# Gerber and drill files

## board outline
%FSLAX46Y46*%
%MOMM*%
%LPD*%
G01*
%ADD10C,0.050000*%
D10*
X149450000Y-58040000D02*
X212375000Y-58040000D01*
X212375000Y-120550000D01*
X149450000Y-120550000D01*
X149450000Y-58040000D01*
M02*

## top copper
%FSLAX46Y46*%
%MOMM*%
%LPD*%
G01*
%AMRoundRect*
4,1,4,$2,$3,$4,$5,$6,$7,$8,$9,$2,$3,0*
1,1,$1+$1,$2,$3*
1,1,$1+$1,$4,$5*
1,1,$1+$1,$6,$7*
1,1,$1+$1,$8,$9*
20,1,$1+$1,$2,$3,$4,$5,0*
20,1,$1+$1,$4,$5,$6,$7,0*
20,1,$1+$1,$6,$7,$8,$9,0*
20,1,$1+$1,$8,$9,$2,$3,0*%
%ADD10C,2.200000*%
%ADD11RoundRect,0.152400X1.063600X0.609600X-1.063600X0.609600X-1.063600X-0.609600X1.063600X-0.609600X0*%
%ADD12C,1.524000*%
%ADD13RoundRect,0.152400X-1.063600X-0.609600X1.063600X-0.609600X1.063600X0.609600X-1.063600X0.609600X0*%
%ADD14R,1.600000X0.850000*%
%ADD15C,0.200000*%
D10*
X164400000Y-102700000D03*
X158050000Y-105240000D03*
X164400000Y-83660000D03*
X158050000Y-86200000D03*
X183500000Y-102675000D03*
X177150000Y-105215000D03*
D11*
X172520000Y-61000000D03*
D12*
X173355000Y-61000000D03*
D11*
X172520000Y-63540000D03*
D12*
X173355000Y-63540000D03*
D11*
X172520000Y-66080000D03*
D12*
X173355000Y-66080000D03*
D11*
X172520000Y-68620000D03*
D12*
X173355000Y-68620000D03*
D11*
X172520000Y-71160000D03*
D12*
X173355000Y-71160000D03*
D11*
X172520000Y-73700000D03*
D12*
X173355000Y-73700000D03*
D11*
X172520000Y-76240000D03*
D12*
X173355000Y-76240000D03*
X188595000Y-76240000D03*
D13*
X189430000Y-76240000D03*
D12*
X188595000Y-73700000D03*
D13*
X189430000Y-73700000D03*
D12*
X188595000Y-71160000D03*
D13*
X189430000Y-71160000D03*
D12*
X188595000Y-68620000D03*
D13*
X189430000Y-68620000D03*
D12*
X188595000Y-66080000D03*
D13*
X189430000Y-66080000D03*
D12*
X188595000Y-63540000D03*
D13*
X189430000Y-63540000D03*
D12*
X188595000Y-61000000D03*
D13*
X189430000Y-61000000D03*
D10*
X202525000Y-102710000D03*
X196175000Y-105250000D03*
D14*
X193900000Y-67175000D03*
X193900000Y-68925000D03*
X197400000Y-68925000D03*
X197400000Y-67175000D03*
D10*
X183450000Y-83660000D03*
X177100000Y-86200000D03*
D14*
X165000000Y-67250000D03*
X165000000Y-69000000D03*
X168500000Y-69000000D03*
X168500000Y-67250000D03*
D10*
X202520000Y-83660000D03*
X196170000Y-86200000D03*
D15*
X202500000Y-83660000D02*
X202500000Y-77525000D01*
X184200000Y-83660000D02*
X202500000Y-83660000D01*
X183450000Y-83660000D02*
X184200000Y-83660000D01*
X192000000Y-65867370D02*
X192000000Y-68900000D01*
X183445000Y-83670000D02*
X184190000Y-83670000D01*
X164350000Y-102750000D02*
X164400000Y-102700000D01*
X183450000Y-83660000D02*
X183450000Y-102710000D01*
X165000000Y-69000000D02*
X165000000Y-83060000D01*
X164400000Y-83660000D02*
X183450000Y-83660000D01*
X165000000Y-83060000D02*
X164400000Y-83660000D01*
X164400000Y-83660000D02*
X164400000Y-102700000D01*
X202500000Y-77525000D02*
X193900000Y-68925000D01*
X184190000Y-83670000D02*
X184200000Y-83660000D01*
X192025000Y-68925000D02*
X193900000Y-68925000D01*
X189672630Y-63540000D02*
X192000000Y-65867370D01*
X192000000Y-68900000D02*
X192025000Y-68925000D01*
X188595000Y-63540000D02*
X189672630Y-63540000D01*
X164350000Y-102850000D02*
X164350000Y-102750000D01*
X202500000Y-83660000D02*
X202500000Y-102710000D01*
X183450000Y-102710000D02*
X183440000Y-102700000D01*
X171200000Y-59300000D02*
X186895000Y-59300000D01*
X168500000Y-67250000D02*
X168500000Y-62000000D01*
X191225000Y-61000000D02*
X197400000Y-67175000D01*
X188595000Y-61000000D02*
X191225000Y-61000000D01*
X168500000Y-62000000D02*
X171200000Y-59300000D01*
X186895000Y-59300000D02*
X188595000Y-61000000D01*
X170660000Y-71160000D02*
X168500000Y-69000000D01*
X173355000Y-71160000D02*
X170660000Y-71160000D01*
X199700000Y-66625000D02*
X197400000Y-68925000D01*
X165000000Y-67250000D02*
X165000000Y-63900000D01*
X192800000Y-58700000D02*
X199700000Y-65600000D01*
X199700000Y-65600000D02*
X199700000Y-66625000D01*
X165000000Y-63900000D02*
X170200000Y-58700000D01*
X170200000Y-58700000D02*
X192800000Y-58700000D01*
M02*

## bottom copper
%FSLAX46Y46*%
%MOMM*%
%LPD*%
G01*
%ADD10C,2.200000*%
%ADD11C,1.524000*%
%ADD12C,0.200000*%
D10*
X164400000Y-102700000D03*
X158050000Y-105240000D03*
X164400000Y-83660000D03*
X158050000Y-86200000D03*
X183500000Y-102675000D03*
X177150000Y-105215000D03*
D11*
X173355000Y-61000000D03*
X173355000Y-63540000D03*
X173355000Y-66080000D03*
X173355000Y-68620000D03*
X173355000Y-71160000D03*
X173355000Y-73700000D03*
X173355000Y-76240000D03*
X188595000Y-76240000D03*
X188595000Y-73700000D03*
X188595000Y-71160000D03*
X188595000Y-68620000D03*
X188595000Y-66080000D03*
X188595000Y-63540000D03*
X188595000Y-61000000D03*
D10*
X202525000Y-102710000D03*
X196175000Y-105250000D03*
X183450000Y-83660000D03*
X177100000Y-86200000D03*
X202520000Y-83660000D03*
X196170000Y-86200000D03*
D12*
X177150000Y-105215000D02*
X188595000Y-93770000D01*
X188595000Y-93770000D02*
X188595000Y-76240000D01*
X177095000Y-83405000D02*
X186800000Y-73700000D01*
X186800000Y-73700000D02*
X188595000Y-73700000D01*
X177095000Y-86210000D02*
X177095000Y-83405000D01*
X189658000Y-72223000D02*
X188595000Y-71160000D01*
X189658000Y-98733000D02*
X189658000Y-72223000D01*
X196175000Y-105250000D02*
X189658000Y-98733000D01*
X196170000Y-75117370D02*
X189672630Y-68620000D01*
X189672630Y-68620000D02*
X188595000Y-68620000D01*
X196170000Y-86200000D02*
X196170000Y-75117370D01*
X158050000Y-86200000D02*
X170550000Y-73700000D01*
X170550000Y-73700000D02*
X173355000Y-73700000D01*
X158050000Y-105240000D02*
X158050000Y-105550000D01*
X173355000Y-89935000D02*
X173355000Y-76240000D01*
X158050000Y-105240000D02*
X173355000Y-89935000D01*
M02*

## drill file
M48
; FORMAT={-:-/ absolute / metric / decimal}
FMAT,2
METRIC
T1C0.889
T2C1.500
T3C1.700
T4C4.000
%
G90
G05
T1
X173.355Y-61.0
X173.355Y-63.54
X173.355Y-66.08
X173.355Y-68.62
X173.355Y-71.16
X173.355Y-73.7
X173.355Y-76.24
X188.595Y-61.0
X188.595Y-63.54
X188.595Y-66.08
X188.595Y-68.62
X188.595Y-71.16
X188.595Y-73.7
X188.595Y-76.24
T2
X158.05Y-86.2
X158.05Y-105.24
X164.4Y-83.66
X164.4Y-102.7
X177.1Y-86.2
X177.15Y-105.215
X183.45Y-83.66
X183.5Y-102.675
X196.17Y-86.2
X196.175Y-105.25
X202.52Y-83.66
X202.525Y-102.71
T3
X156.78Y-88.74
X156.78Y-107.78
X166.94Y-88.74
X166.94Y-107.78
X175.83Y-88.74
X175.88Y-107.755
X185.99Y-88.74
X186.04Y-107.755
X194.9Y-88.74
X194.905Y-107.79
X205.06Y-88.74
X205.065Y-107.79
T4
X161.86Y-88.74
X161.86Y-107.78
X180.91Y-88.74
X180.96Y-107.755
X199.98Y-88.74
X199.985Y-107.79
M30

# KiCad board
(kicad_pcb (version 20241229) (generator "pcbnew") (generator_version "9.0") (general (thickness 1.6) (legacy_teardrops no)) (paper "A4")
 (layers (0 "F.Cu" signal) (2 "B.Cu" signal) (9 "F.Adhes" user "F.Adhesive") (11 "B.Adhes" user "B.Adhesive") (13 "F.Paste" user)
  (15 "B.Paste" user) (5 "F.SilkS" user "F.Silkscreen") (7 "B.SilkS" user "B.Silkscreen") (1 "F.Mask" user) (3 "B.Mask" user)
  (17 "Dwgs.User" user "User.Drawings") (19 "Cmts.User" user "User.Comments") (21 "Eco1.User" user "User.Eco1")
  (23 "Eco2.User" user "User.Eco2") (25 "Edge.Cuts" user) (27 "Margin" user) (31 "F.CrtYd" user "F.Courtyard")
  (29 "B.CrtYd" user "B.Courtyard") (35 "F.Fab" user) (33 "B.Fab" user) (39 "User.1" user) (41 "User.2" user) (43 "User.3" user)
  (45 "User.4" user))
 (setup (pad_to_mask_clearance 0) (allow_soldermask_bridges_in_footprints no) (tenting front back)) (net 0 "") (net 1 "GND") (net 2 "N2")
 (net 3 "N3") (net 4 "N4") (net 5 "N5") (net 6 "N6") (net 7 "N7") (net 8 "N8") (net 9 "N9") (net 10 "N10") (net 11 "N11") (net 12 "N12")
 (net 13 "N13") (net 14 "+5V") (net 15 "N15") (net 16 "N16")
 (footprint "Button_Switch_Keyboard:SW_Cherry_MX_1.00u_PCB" (layer "F.Cu") (at 164.4 102.7)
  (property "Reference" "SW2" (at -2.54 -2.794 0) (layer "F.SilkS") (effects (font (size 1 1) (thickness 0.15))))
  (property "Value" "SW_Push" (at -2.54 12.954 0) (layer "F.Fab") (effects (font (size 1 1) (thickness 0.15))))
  (pad "" np_thru_hole circle (at -7.62 5.08) (size 1.7 1.7) (drill 1.7) (layers "*.Cu" "*.Mask"))
  (pad "" np_thru_hole circle (at -2.54 5.08) (size 4 4) (drill 4) (layers "*.Cu" "*.Mask"))
  (pad "" np_thru_hole circle (at 2.54 5.08) (size 1.7 1.7) (drill 1.7) (layers "*.Cu" "*.Mask"))
  (pad "1" thru_hole circle (at 0 0) (size 2.2 2.2) (drill 1.5) (layers "*.Cu" "*.Mask") (remove_unused_layers no) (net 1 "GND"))
  (pad "2" thru_hole circle (at -6.35 2.54) (size 2.2 2.2) (drill 1.5) (layers "*.Cu" "*.Mask") (remove_unused_layers no) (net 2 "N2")))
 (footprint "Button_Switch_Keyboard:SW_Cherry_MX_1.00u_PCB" (layer "F.Cu") (at 164.4 83.66)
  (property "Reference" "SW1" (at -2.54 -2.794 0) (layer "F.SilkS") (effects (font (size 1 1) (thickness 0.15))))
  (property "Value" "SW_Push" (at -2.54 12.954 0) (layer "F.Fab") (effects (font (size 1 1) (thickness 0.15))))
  (pad "" np_thru_hole circle (at -7.62 5.08) (size 1.7 1.7) (drill 1.7) (layers "*.Cu" "*.Mask"))
  (pad "" np_thru_hole circle (at -2.54 5.08) (size 4 4) (drill 4) (layers "*.Cu" "*.Mask"))
  (pad "" np_thru_hole circle (at 2.54 5.08) (size 1.7 1.7) (drill 1.7) (layers "*.Cu" "*.Mask"))
  (pad "1" thru_hole circle (at 0 0) (size 2.2 2.2) (drill 1.5) (layers "*.Cu" "*.Mask") (remove_unused_layers no) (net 1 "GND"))
  (pad "2" thru_hole circle (at -6.35 2.54) (size 2.2 2.2) (drill 1.5) (layers "*.Cu" "*.Mask") (remove_unused_layers no) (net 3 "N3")))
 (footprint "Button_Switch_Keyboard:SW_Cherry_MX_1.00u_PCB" (layer "F.Cu") (at 183.5 102.675)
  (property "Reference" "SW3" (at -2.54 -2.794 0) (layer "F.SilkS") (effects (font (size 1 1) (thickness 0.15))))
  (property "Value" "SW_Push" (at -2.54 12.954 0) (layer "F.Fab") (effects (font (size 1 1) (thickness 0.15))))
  (pad "" np_thru_hole circle (at -7.62 5.08) (size 1.7 1.7) (drill 1.7) (layers "*.Cu" "*.Mask"))
  (pad "" np_thru_hole circle (at -2.54 5.08) (size 4 4) (drill 4) (layers "*.Cu" "*.Mask"))
  (pad "" np_thru_hole circle (at 2.54 5.08) (size 1.7 1.7) (drill 1.7) (layers "*.Cu" "*.Mask"))
  (pad "1" thru_hole circle (at 0 0) (size 2.2 2.2) (drill 1.5) (layers "*.Cu" "*.Mask") (remove_unused_layers no) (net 1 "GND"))
  (pad "2" thru_hole circle (at -6.35 2.54) (size 2.2 2.2) (drill 1.5) (layers "*.Cu" "*.Mask") (remove_unused_layers no) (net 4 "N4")))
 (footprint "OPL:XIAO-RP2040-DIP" (layer "F.Cu") (at 180.975 68.62)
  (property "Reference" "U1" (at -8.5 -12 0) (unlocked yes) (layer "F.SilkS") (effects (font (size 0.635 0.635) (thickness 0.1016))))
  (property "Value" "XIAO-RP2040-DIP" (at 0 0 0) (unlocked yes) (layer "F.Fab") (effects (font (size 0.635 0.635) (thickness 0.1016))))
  (pad "1" smd roundrect (at -8.455 -7.62 180) (size 2.432 1.524) (layers "F.Cu" "F.Mask") (roundrect_rratio 0.1) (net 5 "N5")
   (thermal_bridge_angle 45))
  (pad "1" thru_hole circle (at -7.62 -7.62 180) (size 1.524 1.524) (drill 0.889) (layers "*.Cu" "*.Mask") (remove_unused_layers no)
   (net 5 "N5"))
  (pad "2" smd roundrect (at -8.455 -5.08 180) (size 2.432 1.524) (layers "F.Cu" "F.Mask") (roundrect_rratio 0.1) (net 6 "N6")
   (thermal_bridge_angle 45))
  (pad "2" thru_hole circle (at -7.62 -5.08 180) (size 1.524 1.524) (drill 0.889) (layers "*.Cu" "*.Mask") (remove_unused_layers no)
   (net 6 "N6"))
  (pad "3" smd roundrect (at -8.455 -2.54 180) (size 2.432 1.524) (layers "F.Cu" "F.Mask") (roundrect_rratio 0.1) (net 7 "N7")
   (thermal_bridge_angle 45))
  (pad "3" thru_hole circle (at -7.62 -2.54 180) (size 1.524 1.524) (drill 0.889) (layers "*.Cu" "*.Mask") (remove_unused_layers no)
   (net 7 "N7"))
  (pad "4" smd roundrect (at -8.455 0 180) (size 2.432 1.524) (layers "F.Cu" "F.Mask") (roundrect_rratio 0.1) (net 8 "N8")
   (thermal_bridge_angle 45))
  (pad "4" thru_hole circle (at -7.62 0 180) (size 1.524 1.524) (drill 0.889) (layers "*.Cu" "*.Mask") (remove_unused_layers no)
   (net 8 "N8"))
  (pad "5" smd roundrect (at -8.455 2.54 180) (size 2.432 1.524) (layers "F.Cu" "F.Mask") (roundrect_rratio 0.1) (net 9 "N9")
   (thermal_bridge_angle 45))
  (pad "5" thru_hole circle (at -7.62 2.54 180) (size 1.524 1.524) (drill 0.889) (layers "*.Cu" "*.Mask") (remove_unused_layers no)
   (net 9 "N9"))
  (pad "6" smd roundrect (at -8.455 5.08 180) (size 2.432 1.524) (layers "F.Cu" "F.Mask") (roundrect_rratio 0.1) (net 3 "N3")
   (thermal_bridge_angle 45))
  (pad "6" thru_hole circle (at -7.62 5.08 180) (size 1.524 1.524) (drill 0.889) (layers "*.Cu" "*.Mask") (remove_unused_layers no)
   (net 3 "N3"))
  (pad "7" smd roundrect (at -8.455 7.62 180) (size 2.432 1.524) (layers "F.Cu" "F.Mask") (roundrect_rratio 0.1) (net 2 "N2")
   (thermal_bridge_angle 45))
  (pad "7" thru_hole circle (at -7.62 7.62 180) (size 1.524 1.524) (drill 0.889) (layers "*.Cu" "*.Mask") (remove_unused_layers no)
   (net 2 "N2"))
  (pad "8" thru_hole circle (at 7.62 7.62) (size 1.524 1.524) (drill 0.889) (layers "*.Cu" "*.Mask") (remove_unused_layers no) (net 4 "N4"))
  (pad "8" smd roundrect (at 8.455 7.62) (size 2.432 1.524) (layers "F.Cu" "F.Mask") (roundrect_rratio 0.1) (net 4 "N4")
   (thermal_bridge_angle 45))
  (pad "9" thru_hole circle (at 7.62 5.08) (size 1.524 1.524) (drill 0.889) (layers "*.Cu" "*.Mask") (remove_unused_layers no)
   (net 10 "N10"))
  (pad "9" smd roundrect (at 8.455 5.08) (size 2.432 1.524) (layers "F.Cu" "F.Mask") (roundrect_rratio 0.1) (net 10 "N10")
   (thermal_bridge_angle 45))
  (pad "10" thru_hole circle (at 7.62 2.54) (size 1.524 1.524) (drill 0.889) (layers "*.Cu" "*.Mask") (remove_unused_layers no)
   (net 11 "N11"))
  (pad "10" smd roundrect (at 8.455 2.54) (size 2.432 1.524) (layers "F.Cu" "F.Mask") (roundrect_rratio 0.1) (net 11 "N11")
   (thermal_bridge_angle 45))
  (pad "11" thru_hole circle (at 7.62 0) (size 1.524 1.524) (drill 0.889) (layers "*.Cu" "*.Mask") (remove_unused_layers no) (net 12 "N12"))
  (pad "11" smd roundrect (at 8.455 0) (size 2.432 1.524) (layers "F.Cu" "F.Mask") (roundrect_rratio 0.1) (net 12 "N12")
   (thermal_bridge_angle 45))
  (pad "12" thru_hole circle (at 7.62 -2.54) (size 1.524 1.524) (drill 0.889) (layers "*.Cu" "*.Mask") (remove_unused_layers no)
   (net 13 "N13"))
  (pad "12" smd roundrect (at 8.455 -2.54) (size 2.432 1.524) (layers "F.Cu" "F.Mask") (roundrect_rratio 0.1) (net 13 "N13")
   (thermal_bridge_angle 45))
  (pad "13" thru_hole circle (at 7.62 -5.08) (size 1.524 1.524) (drill 0.889) (layers "*.Cu" "*.Mask") (remove_unused_layers no)
   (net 1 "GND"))
  (pad "13" smd roundrect (at 8.455 -5.08) (size 2.432 1.524) (layers "F.Cu" "F.Mask") (roundrect_rratio 0.1) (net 1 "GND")
   (thermal_bridge_angle 45))
  (pad "14" thru_hole circle (at 7.62 -7.62) (size 1.524 1.524) (drill 0.889) (layers "*.Cu" "*.Mask") (remove_unused_layers no)
   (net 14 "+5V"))
  (pad "14" smd roundrect (at 8.455 -7.62) (size 2.432 1.524) (layers "F.Cu" "F.Mask") (roundrect_rratio 0.1) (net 14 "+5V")
   (thermal_bridge_angle 45)))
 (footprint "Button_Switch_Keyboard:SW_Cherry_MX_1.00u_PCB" (layer "F.Cu") (at 202.525 102.71)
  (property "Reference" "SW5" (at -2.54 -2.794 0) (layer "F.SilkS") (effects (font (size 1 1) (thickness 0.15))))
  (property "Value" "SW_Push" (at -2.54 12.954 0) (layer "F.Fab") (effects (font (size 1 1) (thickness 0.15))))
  (pad "" np_thru_hole circle (at -7.62 5.08) (size 1.7 1.7) (drill 1.7) (layers "*.Cu" "*.Mask"))
  (pad "" np_thru_hole circle (at -2.54 5.08) (size 4 4) (drill 4) (layers "*.Cu" "*.Mask"))
  (pad "" np_thru_hole circle (at 2.54 5.08) (size 1.7 1.7) (drill 1.7) (layers "*.Cu" "*.Mask"))
  (pad "1" thru_hole circle (at 0 0) (size 2.2 2.2) (drill 1.5) (layers "*.Cu" "*.Mask") (remove_unused_layers no) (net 1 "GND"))
  (pad "2" thru_hole circle (at -6.35 2.54) (size 2.2 2.2) (drill 1.5) (layers "*.Cu" "*.Mask") (remove_unused_layers no) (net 11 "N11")))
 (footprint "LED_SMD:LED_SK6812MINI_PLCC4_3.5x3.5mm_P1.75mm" (layer "F.Cu") (at 195.65 68.05)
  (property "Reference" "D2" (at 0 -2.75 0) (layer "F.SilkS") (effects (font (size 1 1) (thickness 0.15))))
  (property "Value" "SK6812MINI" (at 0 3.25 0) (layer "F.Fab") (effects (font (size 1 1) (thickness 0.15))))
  (pad "1" smd rect (at -1.75 -0.875) (size 1.6 0.85) (layers "F.Cu" "F.Mask" "F.Paste") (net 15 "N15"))
  (pad "2" smd rect (at -1.75 0.875) (size 1.6 0.85) (layers "F.Cu" "F.Mask" "F.Paste") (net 1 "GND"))
  (pad "3" smd rect (at 1.75 0.875) (size 1.6 0.85) (layers "F.Cu" "F.Mask" "F.Paste") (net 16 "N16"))
  (pad "4" smd rect (at 1.75 -0.875) (size 1.6 0.85) (layers "F.Cu" "F.Mask" "F.Paste") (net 14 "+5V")))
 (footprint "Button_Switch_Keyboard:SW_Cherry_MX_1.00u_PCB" (layer "F.Cu") (at 183.45 83.66)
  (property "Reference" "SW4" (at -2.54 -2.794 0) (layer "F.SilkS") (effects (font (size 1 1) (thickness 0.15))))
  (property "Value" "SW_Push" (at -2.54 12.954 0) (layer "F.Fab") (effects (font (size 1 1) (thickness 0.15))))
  (pad "" np_thru_hole circle (at -7.62 5.08) (size 1.7 1.7) (drill 1.7) (layers "*.Cu" "*.Mask"))
  (pad "" np_thru_hole circle (at -2.54 5.08) (size 4 4) (drill 4) (layers "*.Cu" "*.Mask"))
  (pad "" np_thru_hole circle (at 2.54 5.08) (size 1.7 1.7) (drill 1.7) (layers "*.Cu" "*.Mask"))
  (pad "1" thru_hole circle (at 0 0) (size 2.2 2.2) (drill 1.5) (layers "*.Cu" "*.Mask") (remove_unused_layers no) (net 1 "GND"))
  (pad "2" thru_hole circle (at -6.35 2.54) (size 2.2 2.2) (drill 1.5) (layers "*.Cu" "*.Mask") (remove_unused_layers no) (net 10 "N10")))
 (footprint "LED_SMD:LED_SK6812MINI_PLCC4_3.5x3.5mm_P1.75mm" (layer "F.Cu") (at 166.75 68.125)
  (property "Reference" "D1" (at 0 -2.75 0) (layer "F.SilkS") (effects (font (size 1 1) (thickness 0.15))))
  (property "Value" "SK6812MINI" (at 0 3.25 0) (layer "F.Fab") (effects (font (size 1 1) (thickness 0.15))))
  (pad "1" smd rect (at -1.75 -0.875) (size 1.6 0.85) (layers "F.Cu" "F.Mask" "F.Paste") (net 16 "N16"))
  (pad "2" smd rect (at -1.75 0.875) (size 1.6 0.85) (layers "F.Cu" "F.Mask" "F.Paste") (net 1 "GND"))
  (pad "3" smd rect (at 1.75 0.875) (size 1.6 0.85) (layers "F.Cu" "F.Mask" "F.Paste") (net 9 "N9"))
  (pad "4" smd rect (at 1.75 -0.875) (size 1.6 0.85) (layers "F.Cu" "F.Mask" "F.Paste") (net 14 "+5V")))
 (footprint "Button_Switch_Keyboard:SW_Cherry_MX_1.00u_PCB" (layer "F.Cu") (at 202.52 83.66)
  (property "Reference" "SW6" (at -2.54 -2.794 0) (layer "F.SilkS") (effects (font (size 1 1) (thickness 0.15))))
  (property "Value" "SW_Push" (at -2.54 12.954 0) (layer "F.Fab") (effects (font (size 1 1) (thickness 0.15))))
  (pad "" np_thru_hole circle (at -7.62 5.08) (size 1.7 1.7) (drill 1.7) (layers "*.Cu" "*.Mask"))
  (pad "" np_thru_hole circle (at -2.54 5.08) (size 4 4) (drill 4) (layers "*.Cu" "*.Mask"))
  (pad "" np_thru_hole circle (at 2.54 5.08) (size 1.7 1.7) (drill 1.7) (layers "*.Cu" "*.Mask"))
  (pad "1" thru_hole circle (at 0 0) (size 2.2 2.2) (drill 1.5) (layers "*.Cu" "*.Mask") (remove_unused_layers no) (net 1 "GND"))
  (pad "2" thru_hole circle (at -6.35 2.54) (size 2.2 2.2) (drill 1.5) (layers "*.Cu" "*.Mask") (remove_unused_layers no) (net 12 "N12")))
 (gr_rect (start 149.45 58.04) (end 212.375 120.55) (stroke (width 0.05) (type default)) (fill no) (layer "Edge.Cuts"))
 (segment (start 202.5 83.66) (end 202.5 77.525) (width 0.2) (layer "F.Cu") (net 1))
 (segment (start 184.2 83.66) (end 202.5 83.66) (width 0.2) (layer "F.Cu") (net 1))
 (segment (start 183.45 83.66) (end 184.2 83.66) (width 0.2) (layer "F.Cu") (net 1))
 (segment (start 192 65.86737) (end 192 68.9) (width 0.2) (layer "F.Cu") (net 1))
 (segment (start 183.445 83.67) (end 184.19 83.67) (width 0.2) (layer "F.Cu") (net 1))
 (segment (start 164.35 102.75) (end 164.4 102.7) (width 0.2) (layer "F.Cu") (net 1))
 (segment (start 183.45 83.66) (end 183.45 102.71) (width 0.2) (layer "F.Cu") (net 1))
 (segment (start 165 69) (end 165 83.06) (width 0.2) (layer "F.Cu") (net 1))
 (segment (start 164.4 83.66) (end 183.45 83.66) (width 0.2) (layer "F.Cu") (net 1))
 (segment (start 165 83.06) (end 164.4 83.66) (width 0.2) (layer "F.Cu") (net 1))
 (segment (start 164.4 83.66) (end 164.4 102.7) (width 0.2) (layer "F.Cu") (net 1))
 (segment (start 202.5 77.525) (end 193.9 68.925) (width 0.2) (layer "F.Cu") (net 1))
 (segment (start 184.19 83.67) (end 184.2 83.66) (width 0.2) (layer "F.Cu") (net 1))
 (segment (start 192.025 68.925) (end 193.9 68.925) (width 0.2) (layer "F.Cu") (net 1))
 (segment (start 189.67263 63.54) (end 192 65.86737) (width 0.2) (layer "F.Cu") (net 1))
 (segment (start 192 68.9) (end 192.025 68.925) (width 0.2) (layer "F.Cu") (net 1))
 (segment (start 188.595 63.54) (end 189.67263 63.54) (width 0.2) (layer "F.Cu") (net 1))
 (segment (start 164.35 102.85) (end 164.35 102.75) (width 0.2) (layer "F.Cu") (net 1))
 (segment (start 202.5 83.66) (end 202.5 102.71) (width 0.2) (layer "F.Cu") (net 1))
 (segment (start 183.45 102.71) (end 183.44 102.7) (width 0.2) (layer "F.Cu") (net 1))
 (segment (start 171.2 59.3) (end 186.895 59.3) (width 0.2) (layer "F.Cu") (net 14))
 (segment (start 168.5 67.25) (end 168.5 62) (width 0.2) (layer "F.Cu") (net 14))
 (segment (start 191.225 61) (end 197.4 67.175) (width 0.2) (layer "F.Cu") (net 14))
 (segment (start 188.595 61) (end 191.225 61) (width 0.2) (layer "F.Cu") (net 14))
 (segment (start 168.5 62) (end 171.2 59.3) (width 0.2) (layer "F.Cu") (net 14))
 (segment (start 186.895 59.3) (end 188.595 61) (width 0.2) (layer "F.Cu") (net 14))
 (segment (start 170.66 71.16) (end 168.5 69) (width 0.2) (layer "F.Cu") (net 9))
 (segment (start 173.355 71.16) (end 170.66 71.16) (width 0.2) (layer "F.Cu") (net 9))
 (segment (start 199.7 66.625) (end 197.4 68.925) (width 0.2) (layer "F.Cu") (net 16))
 (segment (start 165 67.25) (end 165 63.9) (width 0.2) (layer "F.Cu") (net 16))
 (segment (start 192.8 58.7) (end 199.7 65.6) (width 0.2) (layer "F.Cu") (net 16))
 (segment (start 199.7 65.6) (end 199.7 66.625) (width 0.2) (layer "F.Cu") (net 16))
 (segment (start 165 63.9) (end 170.2 58.7) (width 0.2) (layer "F.Cu") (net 16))
 (segment (start 170.2 58.7) (end 192.8 58.7) (width 0.2) (layer "F.Cu") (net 16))
 (segment (start 177.15 105.215) (end 188.595 93.77) (width 0.2) (layer "B.Cu") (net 4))
 (segment (start 188.595 93.77) (end 188.595 76.24) (width 0.2) (layer "B.Cu") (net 4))
 (segment (start 177.095 83.405) (end 186.8 73.7) (width 0.2) (layer "B.Cu") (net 10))
 (segment (start 186.8 73.7) (end 188.595 73.7) (width 0.2) (layer "B.Cu") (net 10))
 (segment (start 177.095 86.21) (end 177.095 83.405) (width 0.2) (layer "B.Cu") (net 10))
 (segment (start 189.658 72.223) (end 188.595 71.16) (width 0.2) (layer "B.Cu") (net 11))
 (segment (start 189.658 98.733) (end 189.658 72.223) (width 0.2) (layer "B.Cu") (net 11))
 (segment (start 196.175 105.25) (end 189.658 98.733) (width 0.2) (layer "B.Cu") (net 11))
 (segment (start 196.17 75.11737) (end 189.67263 68.62) (width 0.2) (layer "B.Cu") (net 12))
 (segment (start 189.67263 68.62) (end 188.595 68.62) (width 0.2) (layer "B.Cu") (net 12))
 (segment (start 196.17 86.2) (end 196.17 75.11737) (width 0.2) (layer "B.Cu") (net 12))
 (segment (start 158.05 86.2) (end 170.55 73.7) (width 0.2) (layer "B.Cu") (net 3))
 (segment (start 170.55 73.7) (end 173.355 73.7) (width 0.2) (layer "B.Cu") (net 3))
 (segment (start 158.05 105.24) (end 158.05 105.55) (width 0.2) (layer "B.Cu") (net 2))
 (segment (start 173.355 89.935) (end 173.355 76.24) (width 0.2) (layer "B.Cu") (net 2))
 (segment (start 158.05 105.24) (end 173.355 89.935) (width 0.2) (layer "B.Cu") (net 2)))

